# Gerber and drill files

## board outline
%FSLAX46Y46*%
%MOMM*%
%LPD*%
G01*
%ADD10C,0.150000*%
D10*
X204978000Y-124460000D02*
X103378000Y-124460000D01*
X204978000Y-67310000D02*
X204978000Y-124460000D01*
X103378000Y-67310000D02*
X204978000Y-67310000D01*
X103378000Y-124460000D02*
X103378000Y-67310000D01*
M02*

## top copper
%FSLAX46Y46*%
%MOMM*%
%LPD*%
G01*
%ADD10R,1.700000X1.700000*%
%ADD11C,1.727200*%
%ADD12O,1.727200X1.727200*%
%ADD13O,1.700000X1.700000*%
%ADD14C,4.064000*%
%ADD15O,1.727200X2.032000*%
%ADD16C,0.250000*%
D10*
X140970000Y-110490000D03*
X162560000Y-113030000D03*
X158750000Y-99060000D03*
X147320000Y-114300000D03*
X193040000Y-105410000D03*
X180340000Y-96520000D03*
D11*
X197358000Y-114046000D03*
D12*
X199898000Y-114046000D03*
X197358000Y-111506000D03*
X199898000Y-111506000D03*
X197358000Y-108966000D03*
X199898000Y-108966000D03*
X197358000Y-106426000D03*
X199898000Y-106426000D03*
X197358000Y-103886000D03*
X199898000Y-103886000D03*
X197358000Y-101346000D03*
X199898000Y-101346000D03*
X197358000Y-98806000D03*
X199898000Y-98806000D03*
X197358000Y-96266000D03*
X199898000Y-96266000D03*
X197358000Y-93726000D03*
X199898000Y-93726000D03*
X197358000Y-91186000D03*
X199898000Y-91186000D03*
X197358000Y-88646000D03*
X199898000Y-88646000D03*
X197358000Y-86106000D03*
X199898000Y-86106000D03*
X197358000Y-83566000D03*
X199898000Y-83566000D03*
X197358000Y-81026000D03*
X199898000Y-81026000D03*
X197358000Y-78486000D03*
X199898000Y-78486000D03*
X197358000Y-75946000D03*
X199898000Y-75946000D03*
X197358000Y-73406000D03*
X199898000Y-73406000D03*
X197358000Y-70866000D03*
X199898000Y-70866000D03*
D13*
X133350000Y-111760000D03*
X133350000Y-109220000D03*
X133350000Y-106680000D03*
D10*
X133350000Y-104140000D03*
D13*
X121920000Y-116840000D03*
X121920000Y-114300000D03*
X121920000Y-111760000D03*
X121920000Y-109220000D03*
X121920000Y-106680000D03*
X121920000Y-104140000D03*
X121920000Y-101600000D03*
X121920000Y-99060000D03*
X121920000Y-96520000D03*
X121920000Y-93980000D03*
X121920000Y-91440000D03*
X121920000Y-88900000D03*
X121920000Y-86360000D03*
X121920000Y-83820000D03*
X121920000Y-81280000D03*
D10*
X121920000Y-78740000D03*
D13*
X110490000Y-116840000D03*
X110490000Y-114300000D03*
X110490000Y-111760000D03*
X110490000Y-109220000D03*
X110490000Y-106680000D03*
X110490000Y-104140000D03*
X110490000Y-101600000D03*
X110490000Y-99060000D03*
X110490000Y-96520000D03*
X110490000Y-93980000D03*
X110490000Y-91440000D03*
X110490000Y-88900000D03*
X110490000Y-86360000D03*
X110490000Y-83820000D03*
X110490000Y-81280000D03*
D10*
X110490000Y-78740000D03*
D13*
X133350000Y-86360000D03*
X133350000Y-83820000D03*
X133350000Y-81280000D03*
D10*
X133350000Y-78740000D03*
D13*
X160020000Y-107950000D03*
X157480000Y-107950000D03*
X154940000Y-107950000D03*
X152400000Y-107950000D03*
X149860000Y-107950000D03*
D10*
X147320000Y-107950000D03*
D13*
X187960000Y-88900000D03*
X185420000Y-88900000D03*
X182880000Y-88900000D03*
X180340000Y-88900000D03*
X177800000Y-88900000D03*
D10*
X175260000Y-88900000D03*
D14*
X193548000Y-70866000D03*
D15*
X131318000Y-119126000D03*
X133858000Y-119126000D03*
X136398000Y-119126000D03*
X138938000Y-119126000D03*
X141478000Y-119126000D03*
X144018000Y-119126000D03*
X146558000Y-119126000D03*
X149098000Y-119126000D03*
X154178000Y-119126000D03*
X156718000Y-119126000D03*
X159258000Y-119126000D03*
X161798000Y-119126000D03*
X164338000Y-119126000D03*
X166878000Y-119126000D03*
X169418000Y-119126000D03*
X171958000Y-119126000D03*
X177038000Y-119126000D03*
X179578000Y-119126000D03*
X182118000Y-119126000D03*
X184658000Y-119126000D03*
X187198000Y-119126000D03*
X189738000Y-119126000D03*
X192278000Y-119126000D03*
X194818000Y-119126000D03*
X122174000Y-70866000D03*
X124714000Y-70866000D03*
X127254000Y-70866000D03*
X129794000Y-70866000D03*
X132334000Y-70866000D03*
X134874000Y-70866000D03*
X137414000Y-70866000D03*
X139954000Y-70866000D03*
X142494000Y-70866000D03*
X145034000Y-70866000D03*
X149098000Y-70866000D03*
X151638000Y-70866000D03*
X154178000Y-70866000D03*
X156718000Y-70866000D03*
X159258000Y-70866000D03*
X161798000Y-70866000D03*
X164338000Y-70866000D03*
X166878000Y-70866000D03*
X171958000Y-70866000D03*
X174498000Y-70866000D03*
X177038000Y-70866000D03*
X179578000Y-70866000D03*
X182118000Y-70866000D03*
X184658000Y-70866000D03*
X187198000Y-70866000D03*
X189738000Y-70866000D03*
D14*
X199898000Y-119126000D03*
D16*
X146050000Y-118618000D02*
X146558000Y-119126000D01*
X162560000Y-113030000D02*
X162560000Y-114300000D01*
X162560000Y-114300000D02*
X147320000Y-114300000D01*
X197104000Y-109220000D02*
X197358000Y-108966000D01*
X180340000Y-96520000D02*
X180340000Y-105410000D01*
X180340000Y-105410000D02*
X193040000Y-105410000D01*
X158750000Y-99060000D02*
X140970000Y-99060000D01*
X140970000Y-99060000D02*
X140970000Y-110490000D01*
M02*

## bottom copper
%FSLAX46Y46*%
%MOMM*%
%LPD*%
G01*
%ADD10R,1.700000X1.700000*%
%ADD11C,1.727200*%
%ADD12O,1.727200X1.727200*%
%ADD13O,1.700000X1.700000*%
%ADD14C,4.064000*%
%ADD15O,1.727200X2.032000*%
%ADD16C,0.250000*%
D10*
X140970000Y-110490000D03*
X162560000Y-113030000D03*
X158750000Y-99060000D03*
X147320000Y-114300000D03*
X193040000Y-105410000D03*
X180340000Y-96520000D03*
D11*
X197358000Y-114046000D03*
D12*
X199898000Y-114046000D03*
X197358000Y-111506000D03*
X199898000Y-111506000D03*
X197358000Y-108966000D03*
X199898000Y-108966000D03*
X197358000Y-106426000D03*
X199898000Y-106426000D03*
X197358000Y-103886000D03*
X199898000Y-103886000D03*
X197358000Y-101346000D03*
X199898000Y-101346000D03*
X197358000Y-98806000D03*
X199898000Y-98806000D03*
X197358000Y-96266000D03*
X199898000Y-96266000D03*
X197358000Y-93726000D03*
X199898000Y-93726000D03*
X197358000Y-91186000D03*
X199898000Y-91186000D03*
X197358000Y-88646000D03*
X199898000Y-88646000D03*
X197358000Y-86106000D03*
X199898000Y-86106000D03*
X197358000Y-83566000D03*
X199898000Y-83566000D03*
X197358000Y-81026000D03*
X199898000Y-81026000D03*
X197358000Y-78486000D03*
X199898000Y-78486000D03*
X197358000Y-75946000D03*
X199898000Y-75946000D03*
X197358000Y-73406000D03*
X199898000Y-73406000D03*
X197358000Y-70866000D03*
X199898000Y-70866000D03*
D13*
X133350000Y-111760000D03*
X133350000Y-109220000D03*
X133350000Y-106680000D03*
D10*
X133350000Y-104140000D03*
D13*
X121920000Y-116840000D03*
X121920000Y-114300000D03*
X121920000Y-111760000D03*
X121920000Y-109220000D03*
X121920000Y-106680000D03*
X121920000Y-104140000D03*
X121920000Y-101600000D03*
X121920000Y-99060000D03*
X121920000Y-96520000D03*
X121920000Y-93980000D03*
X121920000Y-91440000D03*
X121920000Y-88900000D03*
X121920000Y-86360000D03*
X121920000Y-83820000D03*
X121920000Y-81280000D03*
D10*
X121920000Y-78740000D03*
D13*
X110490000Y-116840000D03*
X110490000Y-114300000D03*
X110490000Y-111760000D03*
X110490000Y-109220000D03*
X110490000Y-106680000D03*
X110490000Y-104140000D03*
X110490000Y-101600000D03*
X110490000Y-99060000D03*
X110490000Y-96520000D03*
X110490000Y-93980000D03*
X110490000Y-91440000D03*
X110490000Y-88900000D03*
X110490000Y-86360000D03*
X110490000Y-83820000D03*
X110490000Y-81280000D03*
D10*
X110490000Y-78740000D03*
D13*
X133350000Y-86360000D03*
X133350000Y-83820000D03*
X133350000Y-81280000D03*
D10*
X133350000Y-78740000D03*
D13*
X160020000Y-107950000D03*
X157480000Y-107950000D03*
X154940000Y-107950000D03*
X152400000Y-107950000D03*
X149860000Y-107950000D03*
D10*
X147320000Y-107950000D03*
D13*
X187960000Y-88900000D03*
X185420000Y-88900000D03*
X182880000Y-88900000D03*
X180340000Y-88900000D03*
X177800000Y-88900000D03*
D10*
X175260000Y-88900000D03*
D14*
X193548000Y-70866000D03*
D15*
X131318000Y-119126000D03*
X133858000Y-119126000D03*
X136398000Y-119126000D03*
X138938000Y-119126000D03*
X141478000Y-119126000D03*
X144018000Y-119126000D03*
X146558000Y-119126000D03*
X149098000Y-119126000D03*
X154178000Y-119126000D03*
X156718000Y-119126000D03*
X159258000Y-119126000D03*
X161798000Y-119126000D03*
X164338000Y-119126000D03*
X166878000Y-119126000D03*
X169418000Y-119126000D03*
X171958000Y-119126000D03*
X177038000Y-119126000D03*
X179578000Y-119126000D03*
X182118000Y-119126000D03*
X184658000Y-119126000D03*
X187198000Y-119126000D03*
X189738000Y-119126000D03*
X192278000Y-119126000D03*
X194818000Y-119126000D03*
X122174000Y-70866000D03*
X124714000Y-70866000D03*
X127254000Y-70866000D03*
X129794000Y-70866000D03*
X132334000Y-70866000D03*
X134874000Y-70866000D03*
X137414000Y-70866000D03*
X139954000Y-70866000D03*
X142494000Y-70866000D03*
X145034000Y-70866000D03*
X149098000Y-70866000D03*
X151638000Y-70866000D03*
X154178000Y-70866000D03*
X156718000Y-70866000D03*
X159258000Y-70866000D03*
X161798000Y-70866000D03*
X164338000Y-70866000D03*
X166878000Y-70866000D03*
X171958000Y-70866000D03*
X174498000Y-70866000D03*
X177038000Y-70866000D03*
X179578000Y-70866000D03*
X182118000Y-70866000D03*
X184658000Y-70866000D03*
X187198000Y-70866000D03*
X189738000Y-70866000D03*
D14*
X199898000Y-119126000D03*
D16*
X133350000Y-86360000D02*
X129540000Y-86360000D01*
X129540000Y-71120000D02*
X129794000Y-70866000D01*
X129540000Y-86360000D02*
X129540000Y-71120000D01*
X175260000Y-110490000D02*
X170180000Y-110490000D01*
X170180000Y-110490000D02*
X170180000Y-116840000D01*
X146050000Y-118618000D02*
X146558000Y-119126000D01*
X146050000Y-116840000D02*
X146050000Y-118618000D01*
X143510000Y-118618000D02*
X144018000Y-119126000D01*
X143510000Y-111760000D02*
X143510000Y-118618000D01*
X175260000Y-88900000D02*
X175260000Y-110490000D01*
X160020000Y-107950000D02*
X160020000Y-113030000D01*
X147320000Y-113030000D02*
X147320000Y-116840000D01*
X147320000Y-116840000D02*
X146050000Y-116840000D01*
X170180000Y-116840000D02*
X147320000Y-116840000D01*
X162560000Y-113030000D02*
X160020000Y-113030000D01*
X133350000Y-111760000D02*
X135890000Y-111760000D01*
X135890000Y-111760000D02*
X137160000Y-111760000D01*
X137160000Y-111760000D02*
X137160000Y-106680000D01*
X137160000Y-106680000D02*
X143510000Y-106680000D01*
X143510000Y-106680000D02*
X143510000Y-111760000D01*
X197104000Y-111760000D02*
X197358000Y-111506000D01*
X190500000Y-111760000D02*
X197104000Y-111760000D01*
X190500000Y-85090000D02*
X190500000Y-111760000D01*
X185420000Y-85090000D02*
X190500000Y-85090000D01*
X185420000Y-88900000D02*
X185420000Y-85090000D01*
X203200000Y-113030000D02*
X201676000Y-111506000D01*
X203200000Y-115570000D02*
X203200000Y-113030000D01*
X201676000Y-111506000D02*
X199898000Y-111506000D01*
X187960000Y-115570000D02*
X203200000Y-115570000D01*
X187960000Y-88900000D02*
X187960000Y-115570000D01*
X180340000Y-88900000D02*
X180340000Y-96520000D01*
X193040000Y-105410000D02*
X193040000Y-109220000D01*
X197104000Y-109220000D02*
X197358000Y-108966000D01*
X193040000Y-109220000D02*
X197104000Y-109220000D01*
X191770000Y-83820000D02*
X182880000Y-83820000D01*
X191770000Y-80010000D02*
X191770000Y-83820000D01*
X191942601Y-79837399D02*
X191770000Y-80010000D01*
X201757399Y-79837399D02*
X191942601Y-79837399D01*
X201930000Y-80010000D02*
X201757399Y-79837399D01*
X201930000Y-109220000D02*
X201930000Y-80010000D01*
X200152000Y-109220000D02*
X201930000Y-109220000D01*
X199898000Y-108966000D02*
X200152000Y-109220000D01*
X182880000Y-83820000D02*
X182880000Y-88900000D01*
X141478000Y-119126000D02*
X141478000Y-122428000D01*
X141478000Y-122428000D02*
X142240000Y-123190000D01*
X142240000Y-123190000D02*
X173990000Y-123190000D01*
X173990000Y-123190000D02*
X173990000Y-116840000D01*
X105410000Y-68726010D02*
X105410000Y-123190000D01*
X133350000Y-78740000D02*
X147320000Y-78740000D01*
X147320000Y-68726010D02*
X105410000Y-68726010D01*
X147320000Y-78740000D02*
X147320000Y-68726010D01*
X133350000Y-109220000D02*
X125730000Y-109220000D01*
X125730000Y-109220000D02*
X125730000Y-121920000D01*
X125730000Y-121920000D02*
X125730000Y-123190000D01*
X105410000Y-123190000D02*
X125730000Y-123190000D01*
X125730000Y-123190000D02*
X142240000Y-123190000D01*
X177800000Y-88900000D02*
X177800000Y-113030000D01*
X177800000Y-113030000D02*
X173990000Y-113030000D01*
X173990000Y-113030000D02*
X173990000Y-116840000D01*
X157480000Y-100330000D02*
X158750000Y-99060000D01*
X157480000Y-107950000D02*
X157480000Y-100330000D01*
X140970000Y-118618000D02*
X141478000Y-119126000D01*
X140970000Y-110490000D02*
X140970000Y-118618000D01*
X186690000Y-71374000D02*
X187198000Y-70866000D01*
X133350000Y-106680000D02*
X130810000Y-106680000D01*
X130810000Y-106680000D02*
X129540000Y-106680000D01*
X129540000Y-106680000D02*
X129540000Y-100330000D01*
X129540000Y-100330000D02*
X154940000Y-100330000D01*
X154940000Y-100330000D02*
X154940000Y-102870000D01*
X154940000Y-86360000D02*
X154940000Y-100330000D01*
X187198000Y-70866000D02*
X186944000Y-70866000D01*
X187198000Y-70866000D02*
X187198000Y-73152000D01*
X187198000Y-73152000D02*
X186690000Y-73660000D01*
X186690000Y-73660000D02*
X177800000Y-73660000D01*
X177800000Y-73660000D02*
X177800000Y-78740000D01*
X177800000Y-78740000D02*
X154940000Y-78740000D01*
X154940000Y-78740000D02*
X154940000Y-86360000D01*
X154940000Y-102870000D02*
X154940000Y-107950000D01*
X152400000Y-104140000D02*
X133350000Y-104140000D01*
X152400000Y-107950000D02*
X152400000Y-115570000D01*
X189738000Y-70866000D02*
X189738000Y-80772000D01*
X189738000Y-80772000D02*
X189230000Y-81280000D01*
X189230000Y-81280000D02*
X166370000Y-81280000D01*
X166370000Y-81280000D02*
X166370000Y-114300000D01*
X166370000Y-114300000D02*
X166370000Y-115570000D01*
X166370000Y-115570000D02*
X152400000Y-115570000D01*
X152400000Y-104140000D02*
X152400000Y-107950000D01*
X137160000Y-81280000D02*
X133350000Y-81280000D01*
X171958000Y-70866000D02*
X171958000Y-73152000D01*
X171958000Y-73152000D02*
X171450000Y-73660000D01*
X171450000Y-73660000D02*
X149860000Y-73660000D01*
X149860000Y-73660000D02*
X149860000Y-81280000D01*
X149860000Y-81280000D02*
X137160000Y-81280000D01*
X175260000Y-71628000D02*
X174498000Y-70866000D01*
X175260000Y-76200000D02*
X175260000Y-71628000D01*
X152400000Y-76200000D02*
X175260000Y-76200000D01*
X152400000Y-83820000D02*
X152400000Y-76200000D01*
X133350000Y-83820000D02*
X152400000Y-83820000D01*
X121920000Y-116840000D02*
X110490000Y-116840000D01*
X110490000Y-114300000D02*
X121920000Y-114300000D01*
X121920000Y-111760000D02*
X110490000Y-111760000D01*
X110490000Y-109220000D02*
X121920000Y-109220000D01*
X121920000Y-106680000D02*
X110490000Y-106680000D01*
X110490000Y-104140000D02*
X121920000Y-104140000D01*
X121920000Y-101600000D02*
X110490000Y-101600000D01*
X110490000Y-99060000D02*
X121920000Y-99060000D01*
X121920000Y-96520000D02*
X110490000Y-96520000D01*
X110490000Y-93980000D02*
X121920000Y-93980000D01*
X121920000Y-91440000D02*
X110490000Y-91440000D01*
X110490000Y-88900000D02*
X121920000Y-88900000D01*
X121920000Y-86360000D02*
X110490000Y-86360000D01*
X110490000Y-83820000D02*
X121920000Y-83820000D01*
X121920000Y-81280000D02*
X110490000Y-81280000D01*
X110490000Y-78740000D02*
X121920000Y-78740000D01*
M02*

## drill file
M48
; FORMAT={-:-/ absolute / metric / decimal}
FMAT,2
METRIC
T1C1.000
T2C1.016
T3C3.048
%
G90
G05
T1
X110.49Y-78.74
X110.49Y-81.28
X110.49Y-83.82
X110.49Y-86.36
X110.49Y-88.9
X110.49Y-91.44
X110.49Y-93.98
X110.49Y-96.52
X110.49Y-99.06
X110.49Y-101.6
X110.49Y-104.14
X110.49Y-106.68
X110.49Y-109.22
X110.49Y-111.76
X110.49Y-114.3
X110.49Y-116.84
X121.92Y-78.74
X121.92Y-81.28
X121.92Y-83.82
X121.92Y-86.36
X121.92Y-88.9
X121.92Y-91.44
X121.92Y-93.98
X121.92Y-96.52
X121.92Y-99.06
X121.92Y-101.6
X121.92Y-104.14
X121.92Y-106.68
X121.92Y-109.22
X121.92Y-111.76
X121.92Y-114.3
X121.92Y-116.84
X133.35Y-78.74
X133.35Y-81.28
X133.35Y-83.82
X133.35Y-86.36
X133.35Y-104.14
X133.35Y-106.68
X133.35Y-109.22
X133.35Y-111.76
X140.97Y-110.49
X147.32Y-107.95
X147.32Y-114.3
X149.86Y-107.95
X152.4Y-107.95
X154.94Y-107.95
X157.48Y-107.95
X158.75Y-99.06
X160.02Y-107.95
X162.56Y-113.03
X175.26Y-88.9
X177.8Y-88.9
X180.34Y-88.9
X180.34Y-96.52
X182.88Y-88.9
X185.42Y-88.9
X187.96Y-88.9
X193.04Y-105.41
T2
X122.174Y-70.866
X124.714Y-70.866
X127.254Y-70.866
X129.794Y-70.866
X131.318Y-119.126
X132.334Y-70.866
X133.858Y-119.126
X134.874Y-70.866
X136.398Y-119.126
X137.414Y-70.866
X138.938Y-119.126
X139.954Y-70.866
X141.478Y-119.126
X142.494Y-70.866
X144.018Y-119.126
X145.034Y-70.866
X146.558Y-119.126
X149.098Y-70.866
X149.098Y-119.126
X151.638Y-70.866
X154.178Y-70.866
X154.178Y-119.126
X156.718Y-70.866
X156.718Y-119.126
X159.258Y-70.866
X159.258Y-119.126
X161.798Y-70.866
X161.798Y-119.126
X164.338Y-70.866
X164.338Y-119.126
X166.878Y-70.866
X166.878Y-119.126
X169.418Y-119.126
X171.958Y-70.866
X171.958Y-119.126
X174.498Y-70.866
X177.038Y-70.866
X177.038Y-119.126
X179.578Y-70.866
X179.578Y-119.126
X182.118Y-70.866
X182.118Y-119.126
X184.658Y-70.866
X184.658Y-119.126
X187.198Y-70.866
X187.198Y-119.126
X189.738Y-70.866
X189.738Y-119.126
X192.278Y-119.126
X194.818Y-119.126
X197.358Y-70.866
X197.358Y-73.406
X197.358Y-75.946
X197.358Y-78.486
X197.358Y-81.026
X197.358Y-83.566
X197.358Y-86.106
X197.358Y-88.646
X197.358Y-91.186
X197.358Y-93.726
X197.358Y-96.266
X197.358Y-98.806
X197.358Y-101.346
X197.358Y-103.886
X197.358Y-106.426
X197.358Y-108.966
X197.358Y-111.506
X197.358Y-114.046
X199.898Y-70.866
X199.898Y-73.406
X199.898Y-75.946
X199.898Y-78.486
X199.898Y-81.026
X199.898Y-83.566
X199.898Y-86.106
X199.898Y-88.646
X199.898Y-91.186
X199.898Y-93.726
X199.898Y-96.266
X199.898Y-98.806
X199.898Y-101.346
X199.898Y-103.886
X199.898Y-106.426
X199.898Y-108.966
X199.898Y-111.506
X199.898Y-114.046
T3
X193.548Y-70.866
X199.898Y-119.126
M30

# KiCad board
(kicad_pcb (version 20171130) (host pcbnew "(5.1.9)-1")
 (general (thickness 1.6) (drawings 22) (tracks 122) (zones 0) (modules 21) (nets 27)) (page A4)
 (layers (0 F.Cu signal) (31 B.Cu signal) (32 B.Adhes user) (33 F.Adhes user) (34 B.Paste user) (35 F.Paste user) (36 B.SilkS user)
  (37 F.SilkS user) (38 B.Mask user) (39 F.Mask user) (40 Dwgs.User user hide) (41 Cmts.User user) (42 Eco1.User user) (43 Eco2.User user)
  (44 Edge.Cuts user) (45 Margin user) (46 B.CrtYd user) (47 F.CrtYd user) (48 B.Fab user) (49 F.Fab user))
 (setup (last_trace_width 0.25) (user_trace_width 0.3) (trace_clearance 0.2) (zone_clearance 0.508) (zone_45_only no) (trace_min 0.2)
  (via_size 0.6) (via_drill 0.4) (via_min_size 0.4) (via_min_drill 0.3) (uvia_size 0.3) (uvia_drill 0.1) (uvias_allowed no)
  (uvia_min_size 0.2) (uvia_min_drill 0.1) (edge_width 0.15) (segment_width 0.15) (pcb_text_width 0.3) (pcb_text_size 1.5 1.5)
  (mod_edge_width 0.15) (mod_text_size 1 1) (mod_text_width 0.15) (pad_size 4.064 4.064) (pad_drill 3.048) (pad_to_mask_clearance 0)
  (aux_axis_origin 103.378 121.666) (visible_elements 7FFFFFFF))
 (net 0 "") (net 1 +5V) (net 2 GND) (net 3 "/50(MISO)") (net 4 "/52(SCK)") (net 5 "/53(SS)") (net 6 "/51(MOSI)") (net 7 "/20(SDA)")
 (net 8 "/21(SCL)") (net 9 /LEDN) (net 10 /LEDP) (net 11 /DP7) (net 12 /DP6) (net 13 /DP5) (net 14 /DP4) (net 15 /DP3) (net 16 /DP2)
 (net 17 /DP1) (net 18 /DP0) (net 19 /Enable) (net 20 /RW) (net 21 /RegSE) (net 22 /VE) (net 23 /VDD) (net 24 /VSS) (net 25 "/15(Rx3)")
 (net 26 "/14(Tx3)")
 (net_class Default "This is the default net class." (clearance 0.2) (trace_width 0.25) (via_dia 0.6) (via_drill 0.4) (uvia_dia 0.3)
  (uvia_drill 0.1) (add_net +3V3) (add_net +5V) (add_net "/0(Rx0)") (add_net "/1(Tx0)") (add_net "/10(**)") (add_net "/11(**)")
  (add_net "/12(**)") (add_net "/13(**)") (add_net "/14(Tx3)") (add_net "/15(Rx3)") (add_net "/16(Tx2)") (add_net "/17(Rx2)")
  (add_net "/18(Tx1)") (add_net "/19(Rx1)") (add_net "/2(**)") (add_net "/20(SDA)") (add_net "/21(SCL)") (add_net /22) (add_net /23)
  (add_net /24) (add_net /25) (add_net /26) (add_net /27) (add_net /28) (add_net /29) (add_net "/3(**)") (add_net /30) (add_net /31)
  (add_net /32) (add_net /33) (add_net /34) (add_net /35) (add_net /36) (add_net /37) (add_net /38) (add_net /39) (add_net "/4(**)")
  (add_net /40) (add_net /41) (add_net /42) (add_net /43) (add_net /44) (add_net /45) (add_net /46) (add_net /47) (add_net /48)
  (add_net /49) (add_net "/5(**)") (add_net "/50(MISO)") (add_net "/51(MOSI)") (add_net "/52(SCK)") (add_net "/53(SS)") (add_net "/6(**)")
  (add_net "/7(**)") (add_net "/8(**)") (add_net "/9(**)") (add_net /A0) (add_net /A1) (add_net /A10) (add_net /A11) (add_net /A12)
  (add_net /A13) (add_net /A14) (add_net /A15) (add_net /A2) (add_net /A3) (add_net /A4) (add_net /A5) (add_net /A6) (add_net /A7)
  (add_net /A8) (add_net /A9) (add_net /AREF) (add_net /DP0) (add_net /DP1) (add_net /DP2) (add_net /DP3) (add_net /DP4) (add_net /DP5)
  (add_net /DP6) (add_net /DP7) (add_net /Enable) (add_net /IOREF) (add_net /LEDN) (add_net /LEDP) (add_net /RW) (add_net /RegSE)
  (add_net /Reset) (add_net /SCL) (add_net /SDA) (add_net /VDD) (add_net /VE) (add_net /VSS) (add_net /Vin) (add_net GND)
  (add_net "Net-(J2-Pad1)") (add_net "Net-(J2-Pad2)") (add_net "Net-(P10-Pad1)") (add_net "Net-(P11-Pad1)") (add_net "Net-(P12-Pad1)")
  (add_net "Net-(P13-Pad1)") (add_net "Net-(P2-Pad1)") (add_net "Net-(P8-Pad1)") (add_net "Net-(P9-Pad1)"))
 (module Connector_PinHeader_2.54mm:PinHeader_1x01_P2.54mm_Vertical (layer F.Cu) (at 140.97 110.49)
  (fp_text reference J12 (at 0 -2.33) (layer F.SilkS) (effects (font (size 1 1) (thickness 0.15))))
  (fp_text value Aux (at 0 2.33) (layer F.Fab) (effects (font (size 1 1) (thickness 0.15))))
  (pad 1 thru_hole rect (at 0 0) (size 1.7 1.7) (drill 1) (layers *.Cu *.Mask) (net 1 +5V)))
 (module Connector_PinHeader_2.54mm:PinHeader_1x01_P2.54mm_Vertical (layer F.Cu) (at 162.56 113.03)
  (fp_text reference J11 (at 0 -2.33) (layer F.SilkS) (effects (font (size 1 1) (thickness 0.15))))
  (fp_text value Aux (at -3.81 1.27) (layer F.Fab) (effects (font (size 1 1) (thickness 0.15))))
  (pad 1 thru_hole rect (at 0 0) (size 1.7 1.7) (drill 1) (layers *.Cu *.Mask) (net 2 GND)))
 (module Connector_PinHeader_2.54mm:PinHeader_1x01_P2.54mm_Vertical (layer F.Cu) (at 158.75 99.06)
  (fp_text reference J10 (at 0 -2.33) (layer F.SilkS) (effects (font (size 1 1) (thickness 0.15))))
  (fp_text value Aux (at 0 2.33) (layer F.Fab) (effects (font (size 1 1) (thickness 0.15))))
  (pad 1 thru_hole rect (at 0 0) (size 1.7 1.7) (drill 1) (layers *.Cu *.Mask) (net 1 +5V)))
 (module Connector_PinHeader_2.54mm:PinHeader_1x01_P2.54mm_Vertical (layer F.Cu) (at 147.32 114.3)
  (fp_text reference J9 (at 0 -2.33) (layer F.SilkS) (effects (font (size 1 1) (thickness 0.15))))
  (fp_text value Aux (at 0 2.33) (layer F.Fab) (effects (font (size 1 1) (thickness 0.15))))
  (pad 1 thru_hole rect (at 0 0) (size 1.7 1.7) (drill 1) (layers *.Cu *.Mask) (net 2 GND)))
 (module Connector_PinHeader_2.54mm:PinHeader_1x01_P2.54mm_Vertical (layer F.Cu) (at 193.04 105.41)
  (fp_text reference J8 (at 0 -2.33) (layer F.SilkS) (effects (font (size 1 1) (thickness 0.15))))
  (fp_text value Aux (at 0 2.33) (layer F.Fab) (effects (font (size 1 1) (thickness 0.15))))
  (pad 1 thru_hole rect (at 0 0) (size 1.7 1.7) (drill 1) (layers *.Cu *.Mask) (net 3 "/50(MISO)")))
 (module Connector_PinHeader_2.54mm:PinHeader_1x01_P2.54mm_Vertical (layer F.Cu) (at 180.34 96.52)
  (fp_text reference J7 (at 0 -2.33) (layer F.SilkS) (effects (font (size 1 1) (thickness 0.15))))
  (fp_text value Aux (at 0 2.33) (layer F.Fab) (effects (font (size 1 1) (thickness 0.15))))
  (pad 1 thru_hole rect (at 0 0) (size 1.7 1.7) (drill 1) (layers *.Cu *.Mask) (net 3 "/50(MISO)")))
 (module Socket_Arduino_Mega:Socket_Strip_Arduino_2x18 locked (layer F.Cu) (at 197.358 114.046 90)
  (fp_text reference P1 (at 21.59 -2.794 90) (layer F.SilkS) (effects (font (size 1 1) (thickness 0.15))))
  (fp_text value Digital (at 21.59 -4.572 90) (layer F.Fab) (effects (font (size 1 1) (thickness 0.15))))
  (pad 1 thru_hole circle (at 0 0 90) (size 1.7272 1.7272) (drill 1.016) (layers *.Cu *.Mask F.SilkS) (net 2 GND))
  (pad 2 thru_hole oval (at 0 2.54 90) (size 1.7272 1.7272) (drill 1.016) (layers *.Cu *.Mask F.SilkS) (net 2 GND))
  (pad 3 thru_hole oval (at 2.54 0 90) (size 1.7272 1.7272) (drill 1.016) (layers *.Cu *.Mask F.SilkS) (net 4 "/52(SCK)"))
  (pad 4 thru_hole oval (at 2.54 2.54 90) (size 1.7272 1.7272) (drill 1.016) (layers *.Cu *.Mask F.SilkS) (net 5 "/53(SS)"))
  (pad 5 thru_hole oval (at 5.08 0 90) (size 1.7272 1.7272) (drill 1.016) (layers *.Cu *.Mask F.SilkS) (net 3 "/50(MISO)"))
  (pad 6 thru_hole oval (at 5.08 2.54 90) (size 1.7272 1.7272) (drill 1.016) (layers *.Cu *.Mask F.SilkS) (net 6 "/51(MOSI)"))
  (pad 7 thru_hole oval (at 7.62 0 90) (size 1.7272 1.7272) (drill 1.016) (layers *.Cu *.Mask F.SilkS))
  (pad 8 thru_hole oval (at 7.62 2.54 90) (size 1.7272 1.7272) (drill 1.016) (layers *.Cu *.Mask F.SilkS))
  (pad 9 thru_hole oval (at 10.16 0 90) (size 1.7272 1.7272) (drill 1.016) (layers *.Cu *.Mask F.SilkS))
  (pad 10 thru_hole oval (at 10.16 2.54 90) (size 1.7272 1.7272) (drill 1.016) (layers *.Cu *.Mask F.SilkS))
  (pad 11 thru_hole oval (at 12.7 0 90) (size 1.7272 1.7272) (drill 1.016) (layers *.Cu *.Mask F.SilkS))
  (pad 12 thru_hole oval (at 12.7 2.54 90) (size 1.7272 1.7272) (drill 1.016) (layers *.Cu *.Mask F.SilkS))
  (pad 13 thru_hole oval (at 15.24 0 90) (size 1.7272 1.7272) (drill 1.016) (layers *.Cu *.Mask F.SilkS))
  (pad 14 thru_hole oval (at 15.24 2.54 90) (size 1.7272 1.7272) (drill 1.016) (layers *.Cu *.Mask F.SilkS))
  (pad 15 thru_hole oval (at 17.78 0 90) (size 1.7272 1.7272) (drill 1.016) (layers *.Cu *.Mask F.SilkS))
  (pad 16 thru_hole oval (at 17.78 2.54 90) (size 1.7272 1.7272) (drill 1.016) (layers *.Cu *.Mask F.SilkS))
  (pad 17 thru_hole oval (at 20.32 0 90) (size 1.7272 1.7272) (drill 1.016) (layers *.Cu *.Mask F.SilkS))
  (pad 18 thru_hole oval (at 20.32 2.54 90) (size 1.7272 1.7272) (drill 1.016) (layers *.Cu *.Mask F.SilkS))
  (pad 19 thru_hole oval (at 22.86 0 90) (size 1.7272 1.7272) (drill 1.016) (layers *.Cu *.Mask F.SilkS))
  (pad 20 thru_hole oval (at 22.86 2.54 90) (size 1.7272 1.7272) (drill 1.016) (layers *.Cu *.Mask F.SilkS))
  (pad 21 thru_hole oval (at 25.4 0 90) (size 1.7272 1.7272) (drill 1.016) (layers *.Cu *.Mask F.SilkS))
  (pad 22 thru_hole oval (at 25.4 2.54 90) (size 1.7272 1.7272) (drill 1.016) (layers *.Cu *.Mask F.SilkS))
  (pad 23 thru_hole oval (at 27.94 0 90) (size 1.7272 1.7272) (drill 1.016) (layers *.Cu *.Mask F.SilkS))
  (pad 24 thru_hole oval (at 27.94 2.54 90) (size 1.7272 1.7272) (drill 1.016) (layers *.Cu *.Mask F.SilkS))
  (pad 25 thru_hole oval (at 30.48 0 90) (size 1.7272 1.7272) (drill 1.016) (layers *.Cu *.Mask F.SilkS))
  (pad 26 thru_hole oval (at 30.48 2.54 90) (size 1.7272 1.7272) (drill 1.016) (layers *.Cu *.Mask F.SilkS))
  (pad 27 thru_hole oval (at 33.02 0 90) (size 1.7272 1.7272) (drill 1.016) (layers *.Cu *.Mask F.SilkS))
  (pad 28 thru_hole oval (at 33.02 2.54 90) (size 1.7272 1.7272) (drill 1.016) (layers *.Cu *.Mask F.SilkS))
  (pad 29 thru_hole oval (at 35.56 0 90) (size 1.7272 1.7272) (drill 1.016) (layers *.Cu *.Mask F.SilkS))
  (pad 30 thru_hole oval (at 35.56 2.54 90) (size 1.7272 1.7272) (drill 1.016) (layers *.Cu *.Mask F.SilkS))
  (pad 31 thru_hole oval (at 38.1 0 90) (size 1.7272 1.7272) (drill 1.016) (layers *.Cu *.Mask F.SilkS))
  (pad 32 thru_hole oval (at 38.1 2.54 90) (size 1.7272 1.7272) (drill 1.016) (layers *.Cu *.Mask F.SilkS))
  (pad 33 thru_hole oval (at 40.64 0 90) (size 1.7272 1.7272) (drill 1.016) (layers *.Cu *.Mask F.SilkS))
  (pad 34 thru_hole oval (at 40.64 2.54 90) (size 1.7272 1.7272) (drill 1.016) (layers *.Cu *.Mask F.SilkS))
  (pad 35 thru_hole oval (at 43.18 0 90) (size 1.7272 1.7272) (drill 1.016) (layers *.Cu *.Mask F.SilkS) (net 1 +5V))
  (pad 36 thru_hole oval (at 43.18 2.54 90) (size 1.7272 1.7272) (drill 1.016) (layers *.Cu *.Mask F.SilkS) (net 1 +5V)))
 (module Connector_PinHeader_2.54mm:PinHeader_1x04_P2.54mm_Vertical (layer F.Cu) (at 133.35 104.14)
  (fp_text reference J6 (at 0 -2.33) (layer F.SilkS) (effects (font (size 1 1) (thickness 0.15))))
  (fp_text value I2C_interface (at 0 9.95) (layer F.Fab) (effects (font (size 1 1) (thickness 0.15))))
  (pad 4 thru_hole oval (at 0 7.62) (size 1.7 1.7) (drill 1) (layers *.Cu *.Mask) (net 2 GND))
  (pad 3 thru_hole oval (at 0 5.08) (size 1.7 1.7) (drill 1) (layers *.Cu *.Mask) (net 1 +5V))
  (pad 2 thru_hole oval (at 0 2.54) (size 1.7 1.7) (drill 1) (layers *.Cu *.Mask) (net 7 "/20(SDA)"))
  (pad 1 thru_hole rect (at 0 0) (size 1.7 1.7) (drill 1) (layers *.Cu *.Mask) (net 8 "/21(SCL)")))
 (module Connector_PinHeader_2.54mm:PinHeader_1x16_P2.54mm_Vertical (layer F.Cu) (at 121.92 78.74)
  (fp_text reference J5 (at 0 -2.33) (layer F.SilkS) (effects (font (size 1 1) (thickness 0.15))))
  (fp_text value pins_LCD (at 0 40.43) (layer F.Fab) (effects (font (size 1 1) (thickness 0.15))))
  (pad 16 thru_hole oval (at 0 38.1) (size 1.7 1.7) (drill 1) (layers *.Cu *.Mask) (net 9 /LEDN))
  (pad 15 thru_hole oval (at 0 35.56) (size 1.7 1.7) (drill 1) (layers *.Cu *.Mask) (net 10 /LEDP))
  (pad 14 thru_hole oval (at 0 33.02) (size 1.7 1.7) (drill 1) (layers *.Cu *.Mask) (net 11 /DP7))
  (pad 13 thru_hole oval (at 0 30.48) (size 1.7 1.7) (drill 1) (layers *.Cu *.Mask) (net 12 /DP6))
  (pad 12 thru_hole oval (at 0 27.94) (size 1.7 1.7) (drill 1) (layers *.Cu *.Mask) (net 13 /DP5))
  (pad 11 thru_hole oval (at 0 25.4) (size 1.7 1.7) (drill 1) (layers *.Cu *.Mask) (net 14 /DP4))
  (pad 10 thru_hole oval (at 0 22.86) (size 1.7 1.7) (drill 1) (layers *.Cu *.Mask) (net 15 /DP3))
  (pad 9 thru_hole oval (at 0 20.32) (size 1.7 1.7) (drill 1) (layers *.Cu *.Mask) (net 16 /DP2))
  (pad 8 thru_hole oval (at 0 17.78) (size 1.7 1.7) (drill 1) (layers *.Cu *.Mask) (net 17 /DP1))
  (pad 7 thru_hole oval (at 0 15.24) (size 1.7 1.7) (drill 1) (layers *.Cu *.Mask) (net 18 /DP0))
  (pad 6 thru_hole oval (at 0 12.7) (size 1.7 1.7) (drill 1) (layers *.Cu *.Mask) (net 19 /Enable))
  (pad 5 thru_hole oval (at 0 10.16) (size 1.7 1.7) (drill 1) (layers *.Cu *.Mask) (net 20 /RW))
  (pad 4 thru_hole oval (at 0 7.62) (size 1.7 1.7) (drill 1) (layers *.Cu *.Mask) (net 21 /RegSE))
  (pad 3 thru_hole oval (at 0 5.08) (size 1.7 1.7) (drill 1) (layers *.Cu *.Mask) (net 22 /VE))
  (pad 2 thru_hole oval (at 0 2.54) (size 1.7 1.7) (drill 1) (layers *.Cu *.Mask) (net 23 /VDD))
  (pad 1 thru_hole rect (at 0 0) (size 1.7 1.7) (drill 1) (layers *.Cu *.Mask) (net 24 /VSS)))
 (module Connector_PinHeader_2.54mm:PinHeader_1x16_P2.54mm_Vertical (layer F.Cu) (at 110.49 78.74)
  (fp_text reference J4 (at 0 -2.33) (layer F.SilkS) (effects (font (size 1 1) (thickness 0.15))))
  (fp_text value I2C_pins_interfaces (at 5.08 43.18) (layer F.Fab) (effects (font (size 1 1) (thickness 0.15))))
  (pad 16 thru_hole oval (at 0 38.1) (size 1.7 1.7) (drill 1) (layers *.Cu *.Mask) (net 9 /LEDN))
  (pad 15 thru_hole oval (at 0 35.56) (size 1.7 1.7) (drill 1) (layers *.Cu *.Mask) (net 10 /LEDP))
  (pad 14 thru_hole oval (at 0 33.02) (size 1.7 1.7) (drill 1) (layers *.Cu *.Mask) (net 11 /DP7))
  (pad 13 thru_hole oval (at 0 30.48) (size 1.7 1.7) (drill 1) (layers *.Cu *.Mask) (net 12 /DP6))
  (pad 12 thru_hole oval (at 0 27.94) (size 1.7 1.7) (drill 1) (layers *.Cu *.Mask) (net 13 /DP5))
  (pad 11 thru_hole oval (at 0 25.4) (size 1.7 1.7) (drill 1) (layers *.Cu *.Mask) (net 14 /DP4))
  (pad 10 thru_hole oval (at 0 22.86) (size 1.7 1.7) (drill 1) (layers *.Cu *.Mask) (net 15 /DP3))
  (pad 9 thru_hole oval (at 0 20.32) (size 1.7 1.7) (drill 1) (layers *.Cu *.Mask) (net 16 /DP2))
  (pad 8 thru_hole oval (at 0 17.78) (size 1.7 1.7) (drill 1) (layers *.Cu *.Mask) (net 17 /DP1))
  (pad 7 thru_hole oval (at 0 15.24) (size 1.7 1.7) (drill 1) (layers *.Cu *.Mask) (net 18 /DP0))
  (pad 6 thru_hole oval (at 0 12.7) (size 1.7 1.7) (drill 1) (layers *.Cu *.Mask) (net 19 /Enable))
  (pad 5 thru_hole oval (at 0 10.16) (size 1.7 1.7) (drill 1) (layers *.Cu *.Mask) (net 20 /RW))
  (pad 4 thru_hole oval (at 0 7.62) (size 1.7 1.7) (drill 1) (layers *.Cu *.Mask) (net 21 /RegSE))
  (pad 3 thru_hole oval (at 0 5.08) (size 1.7 1.7) (drill 1) (layers *.Cu *.Mask) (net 22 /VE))
  (pad 2 thru_hole oval (at 0 2.54) (size 1.7 1.7) (drill 1) (layers *.Cu *.Mask) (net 23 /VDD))
  (pad 1 thru_hole rect (at 0 0) (size 1.7 1.7) (drill 1) (layers *.Cu *.Mask) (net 24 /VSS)))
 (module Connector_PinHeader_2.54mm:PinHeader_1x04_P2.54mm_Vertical (layer F.Cu) (at 133.35 78.74)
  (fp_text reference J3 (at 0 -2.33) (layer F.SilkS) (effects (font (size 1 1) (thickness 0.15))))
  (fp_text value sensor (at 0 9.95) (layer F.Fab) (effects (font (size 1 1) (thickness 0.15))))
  (pad 4 thru_hole oval (at 0 7.62) (size 1.7 1.7) (drill 1) (layers *.Cu *.Mask) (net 2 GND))
  (pad 3 thru_hole oval (at 0 5.08) (size 1.7 1.7) (drill 1) (layers *.Cu *.Mask) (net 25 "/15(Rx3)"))
  (pad 2 thru_hole oval (at 0 2.54) (size 1.7 1.7) (drill 1) (layers *.Cu *.Mask) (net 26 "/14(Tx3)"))
  (pad 1 thru_hole rect (at 0 0) (size 1.7 1.7) (drill 1) (layers *.Cu *.Mask) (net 1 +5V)))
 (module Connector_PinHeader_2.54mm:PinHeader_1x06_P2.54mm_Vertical (layer F.Cu) (at 147.32 107.95 90)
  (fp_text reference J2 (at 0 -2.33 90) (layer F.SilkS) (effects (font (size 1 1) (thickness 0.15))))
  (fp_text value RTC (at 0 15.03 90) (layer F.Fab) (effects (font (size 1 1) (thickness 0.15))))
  (pad 6 thru_hole oval (at 0 12.7 90) (size 1.7 1.7) (drill 1) (layers *.Cu *.Mask) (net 2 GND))
  (pad 5 thru_hole oval (at 0 10.16 90) (size 1.7 1.7) (drill 1) (layers *.Cu *.Mask) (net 1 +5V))
  (pad 4 thru_hole oval (at 0 7.62 90) (size 1.7 1.7) (drill 1) (layers *.Cu *.Mask) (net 7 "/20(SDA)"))
  (pad 3 thru_hole oval (at 0 5.08 90) (size 1.7 1.7) (drill 1) (layers *.Cu *.Mask) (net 8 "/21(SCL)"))
  (pad 2 thru_hole oval (at 0 2.54 90) (size 1.7 1.7) (drill 1) (layers *.Cu *.Mask))
  (pad 1 thru_hole rect (at 0 0 90) (size 1.7 1.7) (drill 1) (layers *.Cu *.Mask)))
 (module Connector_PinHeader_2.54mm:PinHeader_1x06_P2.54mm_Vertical (layer F.Cu) (at 175.26 88.9 90)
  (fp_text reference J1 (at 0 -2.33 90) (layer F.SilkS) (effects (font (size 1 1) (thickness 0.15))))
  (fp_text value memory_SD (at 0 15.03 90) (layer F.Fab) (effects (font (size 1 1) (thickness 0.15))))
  (pad 6 thru_hole oval (at 0 12.7 90) (size 1.7 1.7) (drill 1) (layers *.Cu *.Mask) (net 5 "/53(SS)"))
  (pad 5 thru_hole oval (at 0 10.16 90) (size 1.7 1.7) (drill 1) (layers *.Cu *.Mask) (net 4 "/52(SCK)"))
  (pad 4 thru_hole oval (at 0 7.62 90) (size 1.7 1.7) (drill 1) (layers *.Cu *.Mask) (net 6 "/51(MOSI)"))
  (pad 3 thru_hole oval (at 0 5.08 90) (size 1.7 1.7) (drill 1) (layers *.Cu *.Mask) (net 3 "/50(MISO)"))
  (pad 2 thru_hole oval (at 0 2.54 90) (size 1.7 1.7) (drill 1) (layers *.Cu *.Mask) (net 1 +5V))
  (pad 1 thru_hole rect (at 0 0 90) (size 1.7 1.7) (drill 1) (layers *.Cu *.Mask) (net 2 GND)))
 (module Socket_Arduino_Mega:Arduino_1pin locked (layer F.Cu) (at 193.548 70.866)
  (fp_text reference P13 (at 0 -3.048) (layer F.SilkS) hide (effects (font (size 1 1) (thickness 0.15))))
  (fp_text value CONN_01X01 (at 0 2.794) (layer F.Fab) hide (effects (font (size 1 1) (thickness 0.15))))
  (pad 1 thru_hole circle (at 0 0) (size 4.064 4.064) (drill 3.048) (layers *.Cu *.Mask F.SilkS)))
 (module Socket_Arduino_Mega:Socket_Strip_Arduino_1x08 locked (layer F.Cu) (at 131.318 119.126)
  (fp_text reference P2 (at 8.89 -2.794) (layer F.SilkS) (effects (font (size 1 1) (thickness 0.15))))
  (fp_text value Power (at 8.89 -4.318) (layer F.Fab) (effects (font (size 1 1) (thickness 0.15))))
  (pad 1 thru_hole oval (at 0 0) (size 1.7272 2.032) (drill 1.016) (layers *.Cu *.Mask F.SilkS))
  (pad 2 thru_hole oval (at 2.54 0) (size 1.7272 2.032) (drill 1.016) (layers *.Cu *.Mask F.SilkS))
  (pad 3 thru_hole oval (at 5.08 0) (size 1.7272 2.032) (drill 1.016) (layers *.Cu *.Mask F.SilkS))
  (pad 4 thru_hole oval (at 7.62 0) (size 1.7272 2.032) (drill 1.016) (layers *.Cu *.Mask F.SilkS))
  (pad 5 thru_hole oval (at 10.16 0) (size 1.7272 2.032) (drill 1.016) (layers *.Cu *.Mask F.SilkS) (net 1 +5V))
  (pad 6 thru_hole oval (at 12.7 0) (size 1.7272 2.032) (drill 1.016) (layers *.Cu *.Mask F.SilkS) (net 2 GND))
  (pad 7 thru_hole oval (at 15.24 0) (size 1.7272 2.032) (drill 1.016) (layers *.Cu *.Mask F.SilkS) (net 2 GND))
  (pad 8 thru_hole oval (at 17.78 0) (size 1.7272 2.032) (drill 1.016) (layers *.Cu *.Mask F.SilkS)))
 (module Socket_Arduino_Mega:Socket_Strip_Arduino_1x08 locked (layer F.Cu) (at 154.178 119.126)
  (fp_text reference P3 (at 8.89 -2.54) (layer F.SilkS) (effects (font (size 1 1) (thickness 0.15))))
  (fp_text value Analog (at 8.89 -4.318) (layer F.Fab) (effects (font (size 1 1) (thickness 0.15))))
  (pad 1 thru_hole oval (at 0 0) (size 1.7272 2.032) (drill 1.016) (layers *.Cu *.Mask F.SilkS))
  (pad 2 thru_hole oval (at 2.54 0) (size 1.7272 2.032) (drill 1.016) (layers *.Cu *.Mask F.SilkS))
  (pad 3 thru_hole oval (at 5.08 0) (size 1.7272 2.032) (drill 1.016) (layers *.Cu *.Mask F.SilkS))
  (pad 4 thru_hole oval (at 7.62 0) (size 1.7272 2.032) (drill 1.016) (layers *.Cu *.Mask F.SilkS))
  (pad 5 thru_hole oval (at 10.16 0) (size 1.7272 2.032) (drill 1.016) (layers *.Cu *.Mask F.SilkS))
  (pad 6 thru_hole oval (at 12.7 0) (size 1.7272 2.032) (drill 1.016) (layers *.Cu *.Mask F.SilkS))
  (pad 7 thru_hole oval (at 15.24 0) (size 1.7272 2.032) (drill 1.016) (layers *.Cu *.Mask F.SilkS))
  (pad 8 thru_hole oval (at 17.78 0) (size 1.7272 2.032) (drill 1.016) (layers *.Cu *.Mask F.SilkS)))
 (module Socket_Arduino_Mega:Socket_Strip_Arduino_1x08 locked (layer F.Cu) (at 177.038 119.126)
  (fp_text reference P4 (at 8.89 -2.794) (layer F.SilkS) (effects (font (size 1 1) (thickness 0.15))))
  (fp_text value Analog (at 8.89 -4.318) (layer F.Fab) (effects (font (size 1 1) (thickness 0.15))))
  (pad 1 thru_hole oval (at 0 0) (size 1.7272 2.032) (drill 1.016) (layers *.Cu *.Mask F.SilkS))
  (pad 2 thru_hole oval (at 2.54 0) (size 1.7272 2.032) (drill 1.016) (layers *.Cu *.Mask F.SilkS))
  (pad 3 thru_hole oval (at 5.08 0) (size 1.7272 2.032) (drill 1.016) (layers *.Cu *.Mask F.SilkS))
  (pad 4 thru_hole oval (at 7.62 0) (size 1.7272 2.032) (drill 1.016) (layers *.Cu *.Mask F.SilkS))
  (pad 5 thru_hole oval (at 10.16 0) (size 1.7272 2.032) (drill 1.016) (layers *.Cu *.Mask F.SilkS))
  (pad 6 thru_hole oval (at 12.7 0) (size 1.7272 2.032) (drill 1.016) (layers *.Cu *.Mask F.SilkS))
  (pad 7 thru_hole oval (at 15.24 0) (size 1.7272 2.032) (drill 1.016) (layers *.Cu *.Mask F.SilkS))
  (pad 8 thru_hole oval (at 17.78 0) (size 1.7272 2.032) (drill 1.016) (layers *.Cu *.Mask F.SilkS)))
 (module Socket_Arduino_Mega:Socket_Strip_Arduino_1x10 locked (layer F.Cu) (at 122.174 70.866)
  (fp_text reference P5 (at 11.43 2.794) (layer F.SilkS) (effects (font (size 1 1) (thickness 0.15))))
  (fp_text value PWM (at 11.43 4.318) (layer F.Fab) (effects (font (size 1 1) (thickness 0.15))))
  (pad 1 thru_hole oval (at 0 0) (size 1.7272 2.032) (drill 1.016) (layers *.Cu *.Mask F.SilkS))
  (pad 2 thru_hole oval (at 2.54 0) (size 1.7272 2.032) (drill 1.016) (layers *.Cu *.Mask F.SilkS))
  (pad 3 thru_hole oval (at 5.08 0) (size 1.7272 2.032) (drill 1.016) (layers *.Cu *.Mask F.SilkS))
  (pad 4 thru_hole oval (at 7.62 0) (size 1.7272 2.032) (drill 1.016) (layers *.Cu *.Mask F.SilkS) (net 2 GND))
  (pad 5 thru_hole oval (at 10.16 0) (size 1.7272 2.032) (drill 1.016) (layers *.Cu *.Mask F.SilkS))
  (pad 6 thru_hole oval (at 12.7 0) (size 1.7272 2.032) (drill 1.016) (layers *.Cu *.Mask F.SilkS))
  (pad 7 thru_hole oval (at 15.24 0) (size 1.7272 2.032) (drill 1.016) (layers *.Cu *.Mask F.SilkS))
  (pad 8 thru_hole oval (at 17.78 0) (size 1.7272 2.032) (drill 1.016) (layers *.Cu *.Mask F.SilkS))
  (pad 9 thru_hole oval (at 20.32 0) (size 1.7272 2.032) (drill 1.016) (layers *.Cu *.Mask F.SilkS))
  (pad 10 thru_hole oval (at 22.86 0) (size 1.7272 2.032) (drill 1.016) (layers *.Cu *.Mask F.SilkS)))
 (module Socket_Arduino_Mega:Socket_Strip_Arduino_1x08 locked (layer F.Cu) (at 149.098 70.866)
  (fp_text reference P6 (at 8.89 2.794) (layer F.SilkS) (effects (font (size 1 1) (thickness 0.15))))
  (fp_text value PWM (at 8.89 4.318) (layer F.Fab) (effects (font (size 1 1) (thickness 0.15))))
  (pad 1 thru_hole oval (at 0 0) (size 1.7272 2.032) (drill 1.016) (layers *.Cu *.Mask F.SilkS))
  (pad 2 thru_hole oval (at 2.54 0) (size 1.7272 2.032) (drill 1.016) (layers *.Cu *.Mask F.SilkS))
  (pad 3 thru_hole oval (at 5.08 0) (size 1.7272 2.032) (drill 1.016) (layers *.Cu *.Mask F.SilkS))
  (pad 4 thru_hole oval (at 7.62 0) (size 1.7272 2.032) (drill 1.016) (layers *.Cu *.Mask F.SilkS))
  (pad 5 thru_hole oval (at 10.16 0) (size 1.7272 2.032) (drill 1.016) (layers *.Cu *.Mask F.SilkS))
  (pad 6 thru_hole oval (at 12.7 0) (size 1.7272 2.032) (drill 1.016) (layers *.Cu *.Mask F.SilkS))
  (pad 7 thru_hole oval (at 15.24 0) (size 1.7272 2.032) (drill 1.016) (layers *.Cu *.Mask F.SilkS))
  (pad 8 thru_hole oval (at 17.78 0) (size 1.7272 2.032) (drill 1.016) (layers *.Cu *.Mask F.SilkS)))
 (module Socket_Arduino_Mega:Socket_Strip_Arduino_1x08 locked (layer F.Cu) (at 171.958 70.866)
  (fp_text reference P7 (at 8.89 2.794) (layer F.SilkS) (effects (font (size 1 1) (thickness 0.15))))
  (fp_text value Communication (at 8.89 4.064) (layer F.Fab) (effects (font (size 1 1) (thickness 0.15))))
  (pad 1 thru_hole oval (at 0 0) (size 1.7272 2.032) (drill 1.016) (layers *.Cu *.Mask F.SilkS) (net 26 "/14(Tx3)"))
  (pad 2 thru_hole oval (at 2.54 0) (size 1.7272 2.032) (drill 1.016) (layers *.Cu *.Mask F.SilkS) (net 25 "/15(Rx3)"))
  (pad 3 thru_hole oval (at 5.08 0) (size 1.7272 2.032) (drill 1.016) (layers *.Cu *.Mask F.SilkS))
  (pad 4 thru_hole oval (at 7.62 0) (size 1.7272 2.032) (drill 1.016) (layers *.Cu *.Mask F.SilkS))
  (pad 5 thru_hole oval (at 10.16 0) (size 1.7272 2.032) (drill 1.016) (layers *.Cu *.Mask F.SilkS))
  (pad 6 thru_hole oval (at 12.7 0) (size 1.7272 2.032) (drill 1.016) (layers *.Cu *.Mask F.SilkS))
  (pad 7 thru_hole oval (at 15.24 0) (size 1.7272 2.032) (drill 1.016) (layers *.Cu *.Mask F.SilkS) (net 7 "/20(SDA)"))
  (pad 8 thru_hole oval (at 17.78 0) (size 1.7272 2.032) (drill 1.016) (layers *.Cu *.Mask F.SilkS) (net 8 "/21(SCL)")))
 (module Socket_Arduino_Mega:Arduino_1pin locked (layer F.Cu) (at 199.898 119.126)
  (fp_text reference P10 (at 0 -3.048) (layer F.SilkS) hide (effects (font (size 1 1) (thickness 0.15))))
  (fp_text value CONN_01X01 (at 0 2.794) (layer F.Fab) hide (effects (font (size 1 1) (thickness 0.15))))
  (pad 1 thru_hole circle (at 0 0) (size 4.064 4.064) (drill 3.048) (layers *.Cu *.Mask F.SilkS)))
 (gr_line (start 204.978 124.46) (end 103.378 124.46) (angle 90) (layer Edge.Cuts) (width 0.15))
 (gr_line (start 204.978 67.31) (end 204.978 124.46) (angle 90) (layer Edge.Cuts) (width 0.15))
 (gr_line (start 103.378 67.31) (end 204.978 67.31) (angle 90) (layer Edge.Cuts) (width 0.15))
 (gr_line (start 103.378 124.46) (end 103.378 67.31) (angle 90) (layer Edge.Cuts) (width 0.15))
 (segment (start 133.35 86.36) (end 129.54 86.36) (width 0.25) (layer B.Cu) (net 2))
 (segment (start 129.54 71.12) (end 129.794 70.866) (width 0.25) (layer B.Cu) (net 2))
 (segment (start 129.54 86.36) (end 129.54 71.12) (width 0.25) (layer B.Cu) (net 2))
 (segment (start 175.26 110.49) (end 170.18 110.49) (width 0.25) (layer B.Cu) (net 2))
 (segment (start 170.18 110.49) (end 170.18 116.84) (width 0.25) (layer B.Cu) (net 2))
 (segment (start 146.05 118.618) (end 146.558 119.126) (width 0.25) (layer B.Cu) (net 2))
 (segment (start 146.05 116.84) (end 146.05 118.618) (width 0.25) (layer B.Cu) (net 2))
 (segment (start 143.51 118.618) (end 144.018 119.126) (width 0.25) (layer B.Cu) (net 2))
 (segment (start 143.51 111.76) (end 143.51 118.618) (width 0.25) (layer B.Cu) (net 2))
 (segment (start 146.05 118.618) (end 146.558 119.126) (width 0.25) (layer F.Cu) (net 2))
 (segment (start 175.26 88.9) (end 175.26 110.49) (width 0.25) (layer B.Cu) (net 2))
 (segment (start 160.02 107.95) (end 160.02 113.03) (width 0.25) (layer B.Cu) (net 2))
 (segment (start 147.32 113.03) (end 147.32 116.84) (width 0.25) (layer B.Cu) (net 2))
 (segment (start 147.32 116.84) (end 146.05 116.84) (width 0.25) (layer B.Cu) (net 2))
 (segment (start 170.18 116.84) (end 147.32 116.84) (width 0.25) (layer B.Cu) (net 2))
 (segment (start 162.56 113.03) (end 162.56 114.3) (width 0.25) (layer F.Cu) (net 2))
 (segment (start 162.56 114.3) (end 147.32 114.3) (width 0.25) (layer F.Cu) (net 2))
 (segment (start 162.56 113.03) (end 160.02 113.03) (width 0.25) (layer B.Cu) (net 2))
 (segment (start 133.35 111.76) (end 135.89 111.76) (width 0.25) (layer B.Cu) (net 2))
 (segment (start 135.89 111.76) (end 137.16 111.76) (width 0.25) (layer B.Cu) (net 2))
 (segment (start 137.16 111.76) (end 137.16 106.68) (width 0.25) (layer B.Cu) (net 2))
 (segment (start 137.16 106.68) (end 143.51 106.68) (width 0.25) (layer B.Cu) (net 2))
 (segment (start 143.51 106.68) (end 143.51 111.76) (width 0.25) (layer B.Cu) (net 2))
 (segment (start 197.104 111.76) (end 197.358 111.506) (width 0.25) (layer B.Cu) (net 4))
 (segment (start 190.5 111.76) (end 197.104 111.76) (width 0.25) (layer B.Cu) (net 4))
 (segment (start 190.5 85.09) (end 190.5 111.76) (width 0.25) (layer B.Cu) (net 4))
 (segment (start 185.42 85.09) (end 190.5 85.09) (width 0.25) (layer B.Cu) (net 4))
 (segment (start 185.42 88.9) (end 185.42 85.09) (width 0.25) (layer B.Cu) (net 4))
 (segment (start 203.2 113.03) (end 201.676 111.506) (width 0.25) (layer B.Cu) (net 5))
 (segment (start 203.2 115.57) (end 203.2 113.03) (width 0.25) (layer B.Cu) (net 5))
 (segment (start 201.676 111.506) (end 199.898 111.506) (width 0.25) (layer B.Cu) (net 5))
 (segment (start 187.96 115.57) (end 203.2 115.57) (width 0.25) (layer B.Cu) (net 5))
 (segment (start 187.96 88.9) (end 187.96 115.57) (width 0.25) (layer B.Cu) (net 5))
 (segment (start 197.104 109.22) (end 197.358 108.966) (width 0.25) (layer F.Cu) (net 3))
 (segment (start 180.34 88.9) (end 180.34 96.52) (width 0.25) (layer B.Cu) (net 3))
 (segment (start 193.04 105.41) (end 193.04 109.22) (width 0.25) (layer B.Cu) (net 3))
 (segment (start 197.104 109.22) (end 197.358 108.966) (width 0.25) (layer B.Cu) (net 3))
 (segment (start 193.04 109.22) (end 197.104 109.22) (width 0.25) (layer B.Cu) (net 3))
 (segment (start 180.34 96.52) (end 180.34 105.41) (width 0.25) (layer F.Cu) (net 3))
 (segment (start 180.34 105.41) (end 193.04 105.41) (width 0.25) (layer F.Cu) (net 3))
 (segment (start 191.77 83.82) (end 182.88 83.82) (width 0.25) (layer B.Cu) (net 6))
 (segment (start 191.77 80.01) (end 191.77 83.82) (width 0.25) (layer B.Cu) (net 6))
 (segment (start 191.942601 79.837399) (end 191.77 80.01) (width 0.25) (layer B.Cu) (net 6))
 (segment (start 201.757399 79.837399) (end 191.942601 79.837399) (width 0.25) (layer B.Cu) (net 6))
 (segment (start 201.93 80.01) (end 201.757399 79.837399) (width 0.25) (layer B.Cu) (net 6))
 (segment (start 201.93 109.22) (end 201.93 80.01) (width 0.25) (layer B.Cu) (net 6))
 (segment (start 200.152 109.22) (end 201.93 109.22) (width 0.25) (layer B.Cu) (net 6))
 (segment (start 199.898 108.966) (end 200.152 109.22) (width 0.25) (layer B.Cu) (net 6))
 (segment (start 182.88 83.82) (end 182.88 88.9) (width 0.25) (layer B.Cu) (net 6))
 (segment (start 141.478 119.126) (end 141.478 122.428) (width 0.25) (layer B.Cu) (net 1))
 (segment (start 141.478 122.428) (end 142.24 123.19) (width 0.25) (layer B.Cu) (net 1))
 (segment (start 142.24 123.19) (end 173.99 123.19) (width 0.25) (layer B.Cu) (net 1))
 (segment (start 173.99 123.19) (end 173.99 116.84) (width 0.25) (layer B.Cu) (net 1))
 (segment (start 105.41 68.72601) (end 105.41 123.19) (width 0.25) (layer B.Cu) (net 1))
 (segment (start 133.35 78.74) (end 147.32 78.74) (width 0.25) (layer B.Cu) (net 1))
 (segment (start 147.32 68.72601) (end 105.41 68.72601) (width 0.25) (layer B.Cu) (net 1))
 (segment (start 147.32 78.74) (end 147.32 68.72601) (width 0.25) (layer B.Cu) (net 1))
 (segment (start 133.35 109.22) (end 125.73 109.22) (width 0.25) (layer B.Cu) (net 1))
 (segment (start 125.73 109.22) (end 125.73 121.92) (width 0.25) (layer B.Cu) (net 1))
 (segment (start 125.73 121.92) (end 125.73 123.19) (width 0.25) (layer B.Cu) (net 1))
 (segment (start 105.41 123.19) (end 125.73 123.19) (width 0.25) (layer B.Cu) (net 1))
 (segment (start 125.73 123.19) (end 142.24 123.19) (width 0.25) (layer B.Cu) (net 1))
 (segment (start 177.8 88.9) (end 177.8 113.03) (width 0.25) (layer B.Cu) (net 1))
 (segment (start 177.8 113.03) (end 173.99 113.03) (width 0.25) (layer B.Cu) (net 1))
 (segment (start 173.99 113.03) (end 173.99 116.84) (width 0.25) (layer B.Cu) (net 1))
 (segment (start 157.48 100.33) (end 158.75 99.06) (width 0.25) (layer B.Cu) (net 1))
 (segment (start 157.48 107.95) (end 157.48 100.33) (width 0.25) (layer B.Cu) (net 1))
 (segment (start 140.97 118.618) (end 141.478 119.126) (width 0.25) (layer B.Cu) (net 1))
 (segment (start 140.97 110.49) (end 140.97 118.618) (width 0.25) (layer B.Cu) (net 1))
 (segment (start 158.75 99.06) (end 140.97 99.06) (width 0.25) (layer F.Cu) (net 1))
 (segment (start 140.97 99.06) (end 140.97 110.49) (width 0.25) (layer F.Cu) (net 1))
 (segment (start 186.69 71.374) (end 187.198 70.866) (width 0.25) (layer B.Cu) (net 7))
 (segment (start 133.35 106.68) (end 130.81 106.68) (width 0.25) (layer B.Cu) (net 7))
 (segment (start 130.81 106.68) (end 129.54 106.68) (width 0.25) (layer B.Cu) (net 7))
 (segment (start 129.54 106.68) (end 129.54 100.33) (width 0.25) (layer B.Cu) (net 7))
 (segment (start 129.54 100.33) (end 154.94 100.33) (width 0.25) (layer B.Cu) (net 7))
 (segment (start 154.94 100.33) (end 154.94 102.87) (width 0.25) (layer B.Cu) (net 7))
 (segment (start 154.94 86.36) (end 154.94 100.33) (width 0.25) (layer B.Cu) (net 7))
 (segment (start 187.198 70.866) (end 186.944 70.866) (width 0.25) (layer B.Cu) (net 7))
 (segment (start 187.198 70.866) (end 187.198 73.152) (width 0.25) (layer B.Cu) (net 7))
 (segment (start 187.198 73.152) (end 186.69 73.66) (width 0.25) (layer B.Cu) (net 7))
 (segment (start 186.69 73.66) (end 177.8 73.66) (width 0.25) (layer B.Cu) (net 7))
 (segment (start 177.8 73.66) (end 177.8 78.74) (width 0.25) (layer B.Cu) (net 7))
 (segment (start 177.8 78.74) (end 154.94 78.74) (width 0.25) (layer B.Cu) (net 7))
 (segment (start 154.94 78.74) (end 154.94 86.36) (width 0.25) (layer B.Cu) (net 7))
 (segment (start 154.94 102.87) (end 154.94 107.95) (width 0.25) (layer B.Cu) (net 7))
 (segment (start 152.4 104.14) (end 133.35 104.14) (width 0.25) (layer B.Cu) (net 8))
 (segment (start 152.4 107.95) (end 152.4 115.57) (width 0.25) (layer B.Cu) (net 8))
 (segment (start 189.738 70.866) (end 189.738 80.772) (width 0.25) (layer B.Cu) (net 8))
 (segment (start 189.738 80.772) (end 189.23 81.28) (width 0.25) (layer B.Cu) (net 8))
 (segment (start 189.23 81.28) (end 166.37 81.28) (width 0.25) (layer B.Cu) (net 8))
 (segment (start 166.37 81.28) (end 166.37 114.3) (width 0.25) (layer B.Cu) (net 8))
 (segment (start 166.37 114.3) (end 166.37 115.57) (width 0.25) (layer B.Cu) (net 8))
 (segment (start 166.37 115.57) (end 152.4 115.57) (width 0.25) (layer B.Cu) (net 8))
 (segment (start 152.4 104.14) (end 152.4 107.95) (width 0.25) (layer B.Cu) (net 8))
 (segment (start 137.16 81.28) (end 133.35 81.28) (width 0.25) (layer B.Cu) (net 26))
 (segment (start 171.958 70.866) (end 171.958 73.152) (width 0.25) (layer B.Cu) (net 26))
 (segment (start 171.958 73.152) (end 171.45 73.66) (width 0.25) (layer B.Cu) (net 26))
 (segment (start 171.45 73.66) (end 149.86 73.66) (width 0.25) (layer B.Cu) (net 26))
 (segment (start 149.86 73.66) (end 149.86 81.28) (width 0.25) (layer B.Cu) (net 26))
 (segment (start 149.86 81.28) (end 137.16 81.28) (width 0.25) (layer B.Cu) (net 26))
 (segment (start 175.26 71.628) (end 174.498 70.866) (width 0.25) (layer B.Cu) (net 25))
 (segment (start 175.26 76.2) (end 175.26 71.628) (width 0.25) (layer B.Cu) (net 25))
 (segment (start 152.4 76.2) (end 175.26 76.2) (width 0.25) (layer B.Cu) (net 25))
 (segment (start 152.4 83.82) (end 152.4 76.2) (width 0.25) (layer B.Cu) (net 25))
 (segment (start 133.35 83.82) (end 152.4 83.82) (width 0.25) (layer B.Cu) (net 25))
 (segment (start 121.92 116.84) (end 110.49 116.84) (width 0.25) (layer B.Cu) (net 9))
 (segment (start 110.49 114.3) (end 121.92 114.3) (width 0.25) (layer B.Cu) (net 10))
 (segment (start 121.92 111.76) (end 110.49 111.76) (width 0.25) (layer B.Cu) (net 11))
 (segment (start 110.49 109.22) (end 121.92 109.22) (width 0.25) (layer B.Cu) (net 12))
 (segment (start 121.92 106.68) (end 110.49 106.68) (width 0.25) (layer B.Cu) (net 13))
 (segment (start 110.49 104.14) (end 121.92 104.14) (width 0.25) (layer B.Cu) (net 14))
 (segment (start 121.92 101.6) (end 110.49 101.6) (width 0.25) (layer B.Cu) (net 15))
 (segment (start 110.49 99.06) (end 121.92 99.06) (width 0.25) (layer B.Cu) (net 16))
 (segment (start 121.92 96.52) (end 110.49 96.52) (width 0.25) (layer B.Cu) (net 17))
 (segment (start 110.49 93.98) (end 121.92 93.98) (width 0.25) (layer B.Cu) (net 18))
 (segment (start 121.92 91.44) (end 110.49 91.44) (width 0.25) (layer B.Cu) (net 19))
 (segment (start 110.49 88.9) (end 121.92 88.9) (width 0.25) (layer B.Cu) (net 20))
 (segment (start 121.92 86.36) (end 110.49 86.36) (width 0.25) (layer B.Cu) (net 21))
 (segment (start 110.49 83.82) (end 121.92 83.82) (width 0.25) (layer B.Cu) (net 22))
 (segment (start 121.92 81.28) (end 110.49 81.28) (width 0.25) (layer B.Cu) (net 23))
 (segment (start 110.49 78.74) (end 121.92 78.74) (width 0.25) (layer B.Cu) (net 24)))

